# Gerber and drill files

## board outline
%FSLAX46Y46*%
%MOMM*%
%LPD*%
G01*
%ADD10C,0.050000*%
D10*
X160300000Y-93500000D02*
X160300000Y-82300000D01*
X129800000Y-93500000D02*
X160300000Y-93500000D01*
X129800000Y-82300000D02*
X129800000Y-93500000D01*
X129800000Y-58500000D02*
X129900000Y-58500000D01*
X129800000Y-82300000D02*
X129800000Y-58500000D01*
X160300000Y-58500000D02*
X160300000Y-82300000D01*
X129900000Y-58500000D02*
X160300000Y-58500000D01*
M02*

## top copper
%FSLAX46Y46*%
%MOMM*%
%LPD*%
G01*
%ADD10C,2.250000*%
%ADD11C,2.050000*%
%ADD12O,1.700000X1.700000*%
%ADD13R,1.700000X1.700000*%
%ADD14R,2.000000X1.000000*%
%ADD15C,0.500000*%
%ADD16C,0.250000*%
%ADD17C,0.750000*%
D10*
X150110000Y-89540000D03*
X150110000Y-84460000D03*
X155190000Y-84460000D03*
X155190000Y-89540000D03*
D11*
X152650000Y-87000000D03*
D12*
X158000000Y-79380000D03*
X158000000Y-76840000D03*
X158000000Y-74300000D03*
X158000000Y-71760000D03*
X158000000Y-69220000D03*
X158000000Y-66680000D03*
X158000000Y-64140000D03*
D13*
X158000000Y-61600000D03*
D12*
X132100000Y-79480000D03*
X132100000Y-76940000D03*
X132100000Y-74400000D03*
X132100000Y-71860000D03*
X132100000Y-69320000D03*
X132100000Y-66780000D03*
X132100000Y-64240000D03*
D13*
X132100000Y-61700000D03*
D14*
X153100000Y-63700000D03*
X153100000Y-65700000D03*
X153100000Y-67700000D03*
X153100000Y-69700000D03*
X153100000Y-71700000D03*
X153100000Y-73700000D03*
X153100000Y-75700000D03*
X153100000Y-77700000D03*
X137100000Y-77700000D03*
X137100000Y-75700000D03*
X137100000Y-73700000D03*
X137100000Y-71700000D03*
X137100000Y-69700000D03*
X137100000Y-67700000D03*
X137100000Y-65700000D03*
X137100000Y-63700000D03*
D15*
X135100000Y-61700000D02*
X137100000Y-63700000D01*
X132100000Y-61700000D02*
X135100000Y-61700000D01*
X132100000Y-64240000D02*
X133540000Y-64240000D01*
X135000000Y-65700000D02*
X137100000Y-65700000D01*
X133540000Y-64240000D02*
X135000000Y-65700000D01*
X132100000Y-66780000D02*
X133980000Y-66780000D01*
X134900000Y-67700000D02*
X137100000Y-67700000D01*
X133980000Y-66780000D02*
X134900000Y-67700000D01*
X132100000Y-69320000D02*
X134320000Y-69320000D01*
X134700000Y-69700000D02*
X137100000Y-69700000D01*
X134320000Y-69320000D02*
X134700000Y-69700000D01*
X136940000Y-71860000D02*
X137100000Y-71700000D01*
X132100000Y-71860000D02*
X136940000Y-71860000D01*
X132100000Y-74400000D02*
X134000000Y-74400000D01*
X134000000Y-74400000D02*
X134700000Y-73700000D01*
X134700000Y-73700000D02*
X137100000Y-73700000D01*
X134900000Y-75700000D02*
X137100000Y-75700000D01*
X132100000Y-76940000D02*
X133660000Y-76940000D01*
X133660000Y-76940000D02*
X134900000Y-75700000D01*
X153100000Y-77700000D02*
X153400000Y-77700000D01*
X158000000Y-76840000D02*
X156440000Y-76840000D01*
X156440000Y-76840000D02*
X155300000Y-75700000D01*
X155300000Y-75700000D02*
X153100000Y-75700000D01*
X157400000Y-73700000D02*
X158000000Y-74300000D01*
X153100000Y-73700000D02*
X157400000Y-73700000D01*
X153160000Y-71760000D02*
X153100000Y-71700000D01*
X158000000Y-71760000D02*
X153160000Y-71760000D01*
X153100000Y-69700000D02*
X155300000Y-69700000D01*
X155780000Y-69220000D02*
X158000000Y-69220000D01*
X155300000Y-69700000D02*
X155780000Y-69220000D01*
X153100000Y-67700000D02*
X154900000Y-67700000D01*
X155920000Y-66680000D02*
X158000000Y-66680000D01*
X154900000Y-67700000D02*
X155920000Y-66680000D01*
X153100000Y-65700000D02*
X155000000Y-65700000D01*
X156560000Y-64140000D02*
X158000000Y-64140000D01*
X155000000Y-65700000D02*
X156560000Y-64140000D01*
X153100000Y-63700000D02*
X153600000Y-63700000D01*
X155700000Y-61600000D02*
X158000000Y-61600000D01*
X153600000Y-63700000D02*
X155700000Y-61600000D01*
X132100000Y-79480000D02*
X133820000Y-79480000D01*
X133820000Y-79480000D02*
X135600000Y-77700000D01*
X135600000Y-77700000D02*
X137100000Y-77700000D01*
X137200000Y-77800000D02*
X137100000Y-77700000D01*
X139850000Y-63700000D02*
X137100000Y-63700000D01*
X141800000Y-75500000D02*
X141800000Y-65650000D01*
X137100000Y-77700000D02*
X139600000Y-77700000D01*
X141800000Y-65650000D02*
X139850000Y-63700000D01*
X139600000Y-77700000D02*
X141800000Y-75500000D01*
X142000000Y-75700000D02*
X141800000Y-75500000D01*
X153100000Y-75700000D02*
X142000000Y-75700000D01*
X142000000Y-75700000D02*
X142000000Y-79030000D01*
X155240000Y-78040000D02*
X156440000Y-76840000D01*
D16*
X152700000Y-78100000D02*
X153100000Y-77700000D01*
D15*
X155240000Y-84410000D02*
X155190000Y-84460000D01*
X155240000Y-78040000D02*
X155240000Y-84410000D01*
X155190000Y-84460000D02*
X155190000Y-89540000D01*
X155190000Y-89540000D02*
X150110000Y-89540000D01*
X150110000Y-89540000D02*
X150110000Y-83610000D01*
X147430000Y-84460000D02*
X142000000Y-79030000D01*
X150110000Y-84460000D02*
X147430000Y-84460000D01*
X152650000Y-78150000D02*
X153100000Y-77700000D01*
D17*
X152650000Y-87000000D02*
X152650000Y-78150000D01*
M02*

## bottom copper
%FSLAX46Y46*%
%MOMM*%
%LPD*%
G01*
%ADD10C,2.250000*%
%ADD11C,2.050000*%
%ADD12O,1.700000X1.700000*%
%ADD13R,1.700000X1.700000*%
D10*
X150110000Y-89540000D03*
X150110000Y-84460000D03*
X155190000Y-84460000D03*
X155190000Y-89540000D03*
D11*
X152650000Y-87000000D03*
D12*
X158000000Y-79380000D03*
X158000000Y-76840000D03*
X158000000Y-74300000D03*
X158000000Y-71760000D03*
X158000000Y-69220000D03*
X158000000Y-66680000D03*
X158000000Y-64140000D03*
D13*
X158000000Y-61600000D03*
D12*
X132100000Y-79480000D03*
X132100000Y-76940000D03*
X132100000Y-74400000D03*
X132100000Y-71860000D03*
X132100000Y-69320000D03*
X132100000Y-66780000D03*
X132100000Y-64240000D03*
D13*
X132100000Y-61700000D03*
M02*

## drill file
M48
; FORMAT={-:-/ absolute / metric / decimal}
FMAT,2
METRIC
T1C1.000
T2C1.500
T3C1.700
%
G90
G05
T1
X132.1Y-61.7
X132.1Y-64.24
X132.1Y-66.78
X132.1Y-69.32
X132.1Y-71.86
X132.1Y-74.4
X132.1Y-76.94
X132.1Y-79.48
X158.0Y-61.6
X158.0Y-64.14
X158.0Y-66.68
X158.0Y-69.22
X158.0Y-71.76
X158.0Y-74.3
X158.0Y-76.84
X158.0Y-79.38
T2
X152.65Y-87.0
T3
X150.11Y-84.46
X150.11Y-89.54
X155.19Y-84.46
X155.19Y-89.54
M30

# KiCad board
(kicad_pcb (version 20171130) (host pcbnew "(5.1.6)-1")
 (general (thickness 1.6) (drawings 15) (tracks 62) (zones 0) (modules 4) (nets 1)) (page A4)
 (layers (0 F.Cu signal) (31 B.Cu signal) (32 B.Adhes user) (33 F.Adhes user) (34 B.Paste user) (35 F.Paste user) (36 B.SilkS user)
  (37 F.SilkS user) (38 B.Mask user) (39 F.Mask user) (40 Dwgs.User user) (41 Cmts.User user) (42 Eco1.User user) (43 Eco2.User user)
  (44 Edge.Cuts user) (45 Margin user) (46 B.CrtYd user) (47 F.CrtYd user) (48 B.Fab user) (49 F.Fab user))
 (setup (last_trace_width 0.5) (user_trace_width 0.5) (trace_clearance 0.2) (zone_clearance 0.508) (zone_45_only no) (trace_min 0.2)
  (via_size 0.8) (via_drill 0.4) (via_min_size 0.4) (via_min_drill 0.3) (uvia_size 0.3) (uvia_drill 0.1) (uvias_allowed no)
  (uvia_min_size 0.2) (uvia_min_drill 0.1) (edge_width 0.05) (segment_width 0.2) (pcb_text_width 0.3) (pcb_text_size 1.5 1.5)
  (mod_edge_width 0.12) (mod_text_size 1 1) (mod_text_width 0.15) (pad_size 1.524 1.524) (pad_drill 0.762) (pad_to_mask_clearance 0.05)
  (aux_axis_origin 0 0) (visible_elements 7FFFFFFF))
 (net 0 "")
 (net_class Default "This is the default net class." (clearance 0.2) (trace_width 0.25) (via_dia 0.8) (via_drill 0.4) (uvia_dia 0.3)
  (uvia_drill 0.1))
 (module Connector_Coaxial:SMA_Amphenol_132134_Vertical (layer F.Cu) (at 152.65 87)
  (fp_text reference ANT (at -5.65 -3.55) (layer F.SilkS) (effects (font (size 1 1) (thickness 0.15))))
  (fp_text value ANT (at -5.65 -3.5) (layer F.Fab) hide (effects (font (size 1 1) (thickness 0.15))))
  (pad 2 thru_hole circle (at -2.54 2.54) (size 2.25 2.25) (drill 1.7) (layers *.Cu *.Mask))
  (pad 2 thru_hole circle (at -2.54 -2.54) (size 2.25 2.25) (drill 1.7) (layers *.Cu *.Mask))
  (pad 2 thru_hole circle (at 2.54 -2.54) (size 2.25 2.25) (drill 1.7) (layers *.Cu *.Mask))
  (pad 2 thru_hole circle (at 2.54 2.54) (size 2.25 2.25) (drill 1.7) (layers *.Cu *.Mask))
  (pad 1 thru_hole circle (at 0 0) (size 2.05 2.05) (drill 1.5) (layers *.Cu *.Mask)))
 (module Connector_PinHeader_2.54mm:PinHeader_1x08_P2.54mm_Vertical (layer F.Cu) (at 158 61.6)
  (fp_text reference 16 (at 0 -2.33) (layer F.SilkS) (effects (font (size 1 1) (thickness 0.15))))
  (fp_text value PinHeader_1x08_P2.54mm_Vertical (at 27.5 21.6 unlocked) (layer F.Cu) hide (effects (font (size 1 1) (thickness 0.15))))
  (pad 8 thru_hole oval (at 0 17.78) (size 1.7 1.7) (drill 1) (layers *.Cu *.Mask))
  (pad 7 thru_hole oval (at 0 15.24) (size 1.7 1.7) (drill 1) (layers *.Cu *.Mask))
  (pad 6 thru_hole oval (at 0 12.7) (size 1.7 1.7) (drill 1) (layers *.Cu *.Mask))
  (pad 5 thru_hole oval (at 0 10.16) (size 1.7 1.7) (drill 1) (layers *.Cu *.Mask))
  (pad 4 thru_hole oval (at 0 7.62) (size 1.7 1.7) (drill 1) (layers *.Cu *.Mask))
  (pad 3 thru_hole oval (at 0 5.08) (size 1.7 1.7) (drill 1) (layers *.Cu *.Mask))
  (pad 2 thru_hole oval (at 0 2.54) (size 1.7 1.7) (drill 1) (layers *.Cu *.Mask))
  (pad 1 thru_hole rect (at 0 0) (size 1.7 1.7) (drill 1) (layers *.Cu *.Mask)))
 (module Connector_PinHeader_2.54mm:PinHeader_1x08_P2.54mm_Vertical (layer F.Cu) (at 132.1 61.7)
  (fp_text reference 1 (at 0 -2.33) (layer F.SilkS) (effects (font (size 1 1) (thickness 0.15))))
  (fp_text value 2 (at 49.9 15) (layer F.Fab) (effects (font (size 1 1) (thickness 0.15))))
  (pad 8 thru_hole oval (at 0 17.78) (size 1.7 1.7) (drill 1) (layers *.Cu *.Mask))
  (pad 7 thru_hole oval (at 0 15.24) (size 1.7 1.7) (drill 1) (layers *.Cu *.Mask))
  (pad 6 thru_hole oval (at 0 12.7) (size 1.7 1.7) (drill 1) (layers *.Cu *.Mask))
  (pad 5 thru_hole oval (at 0 10.16) (size 1.7 1.7) (drill 1) (layers *.Cu *.Mask))
  (pad 4 thru_hole oval (at 0 7.62) (size 1.7 1.7) (drill 1) (layers *.Cu *.Mask))
  (pad 3 thru_hole oval (at 0 5.08) (size 1.7 1.7) (drill 1) (layers *.Cu *.Mask))
  (pad 2 thru_hole oval (at 0 2.54) (size 1.7 1.7) (drill 1) (layers *.Cu *.Mask))
  (pad 1 thru_hole rect (at 0 0) (size 1.7 1.7) (drill 1) (layers *.Cu *.Mask)))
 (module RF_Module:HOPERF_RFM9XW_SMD (layer F.Cu) (at 145.1 70.7)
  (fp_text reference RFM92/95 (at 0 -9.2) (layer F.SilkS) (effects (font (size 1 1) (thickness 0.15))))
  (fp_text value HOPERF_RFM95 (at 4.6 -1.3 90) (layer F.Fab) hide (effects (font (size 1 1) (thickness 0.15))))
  (pad 16 smd rect (at 8 -7) (size 2 1) (layers F.Cu F.Paste F.Mask))
  (pad 15 smd rect (at 8 -5) (size 2 1) (layers F.Cu F.Paste F.Mask))
  (pad 14 smd rect (at 8 -3) (size 2 1) (layers F.Cu F.Paste F.Mask))
  (pad 13 smd rect (at 8 -1) (size 2 1) (layers F.Cu F.Paste F.Mask))
  (pad 12 smd rect (at 8 1) (size 2 1) (layers F.Cu F.Paste F.Mask))
  (pad 11 smd rect (at 8 3) (size 2 1) (layers F.Cu F.Paste F.Mask))
  (pad 10 smd rect (at 8 5) (size 2 1) (layers F.Cu F.Paste F.Mask))
  (pad 9 smd rect (at 8 7) (size 2 1) (layers F.Cu F.Paste F.Mask))
  (pad 8 smd rect (at -8 7) (size 2 1) (layers F.Cu F.Paste F.Mask))
  (pad 7 smd rect (at -8 5) (size 2 1) (layers F.Cu F.Paste F.Mask))
  (pad 6 smd rect (at -8 3) (size 2 1) (layers F.Cu F.Paste F.Mask))
  (pad 5 smd rect (at -8 1) (size 2 1) (layers F.Cu F.Paste F.Mask))
  (pad 4 smd rect (at -8 -1) (size 2 1) (layers F.Cu F.Paste F.Mask))
  (pad 3 smd rect (at -8 -3) (size 2 1) (layers F.Cu F.Paste F.Mask))
  (pad 2 smd rect (at -8 -5) (size 2 1) (layers F.Cu F.Paste F.Mask))
  (pad 1 smd rect (at -8 -7) (size 2 1) (layers F.Cu F.Paste F.Mask)))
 (gr_line (start 160.3 93.5) (end 160.3 82.3) (layer Edge.Cuts) (width 0.05))
 (gr_line (start 129.8 93.5) (end 160.3 93.5) (layer Edge.Cuts) (width 0.05))
 (gr_line (start 129.8 82.3) (end 129.8 93.5) (layer Edge.Cuts) (width 0.05))
 (gr_line (start 129.8 58.5) (end 129.9 58.5) (layer Edge.Cuts) (width 0.05))
 (gr_line (start 129.8 82.3) (end 129.8 58.5) (layer Edge.Cuts) (width 0.05))
 (gr_line (start 160.3 58.5) (end 160.3 82.3) (layer Edge.Cuts) (width 0.05))
 (gr_line (start 129.9 58.5) (end 160.3 58.5) (layer Edge.Cuts) (width 0.05))
 (segment (start 135.1 61.7) (end 137.1 63.7) (width 0.5) (layer F.Cu) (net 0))
 (segment (start 132.1 61.7) (end 135.1 61.7) (width 0.5) (layer F.Cu) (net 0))
 (segment (start 132.1 64.24) (end 133.54 64.24) (width 0.5) (layer F.Cu) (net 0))
 (segment (start 135 65.7) (end 137.1 65.7) (width 0.5) (layer F.Cu) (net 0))
 (segment (start 133.54 64.24) (end 135 65.7) (width 0.5) (layer F.Cu) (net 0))
 (segment (start 132.1 66.78) (end 133.98 66.78) (width 0.5) (layer F.Cu) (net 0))
 (segment (start 134.9 67.7) (end 137.1 67.7) (width 0.5) (layer F.Cu) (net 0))
 (segment (start 133.98 66.78) (end 134.9 67.7) (width 0.5) (layer F.Cu) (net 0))
 (segment (start 132.1 69.32) (end 134.32 69.32) (width 0.5) (layer F.Cu) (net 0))
 (segment (start 134.7 69.7) (end 137.1 69.7) (width 0.5) (layer F.Cu) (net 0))
 (segment (start 134.32 69.32) (end 134.7 69.7) (width 0.5) (layer F.Cu) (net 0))
 (segment (start 136.94 71.86) (end 137.1 71.7) (width 0.5) (layer F.Cu) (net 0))
 (segment (start 132.1 71.86) (end 136.94 71.86) (width 0.5) (layer F.Cu) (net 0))
 (segment (start 132.1 74.4) (end 134 74.4) (width 0.5) (layer F.Cu) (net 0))
 (segment (start 134 74.4) (end 134.7 73.7) (width 0.5) (layer F.Cu) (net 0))
 (segment (start 134.7 73.7) (end 137.1 73.7) (width 0.5) (layer F.Cu) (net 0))
 (segment (start 134.9 75.7) (end 137.1 75.7) (width 0.5) (layer F.Cu) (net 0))
 (segment (start 132.1 76.94) (end 133.66 76.94) (width 0.5) (layer F.Cu) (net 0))
 (segment (start 133.66 76.94) (end 134.9 75.7) (width 0.5) (layer F.Cu) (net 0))
 (segment (start 153.1 77.7) (end 153.4 77.7) (width 0.5) (layer F.Cu) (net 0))
 (segment (start 158 76.84) (end 156.44 76.84) (width 0.5) (layer F.Cu) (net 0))
 (segment (start 156.44 76.84) (end 155.3 75.7) (width 0.5) (layer F.Cu) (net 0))
 (segment (start 155.3 75.7) (end 153.1 75.7) (width 0.5) (layer F.Cu) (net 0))
 (segment (start 157.4 73.7) (end 158 74.3) (width 0.5) (layer F.Cu) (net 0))
 (segment (start 153.1 73.7) (end 157.4 73.7) (width 0.5) (layer F.Cu) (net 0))
 (segment (start 153.16 71.76) (end 153.1 71.7) (width 0.5) (layer F.Cu) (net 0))
 (segment (start 158 71.76) (end 153.16 71.76) (width 0.5) (layer F.Cu) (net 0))
 (segment (start 153.1 69.7) (end 155.3 69.7) (width 0.5) (layer F.Cu) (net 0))
 (segment (start 155.78 69.22) (end 158 69.22) (width 0.5) (layer F.Cu) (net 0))
 (segment (start 155.3 69.7) (end 155.78 69.22) (width 0.5) (layer F.Cu) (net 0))
 (segment (start 153.1 67.7) (end 154.9 67.7) (width 0.5) (layer F.Cu) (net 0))
 (segment (start 155.92 66.68) (end 158 66.68) (width 0.5) (layer F.Cu) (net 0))
 (segment (start 154.9 67.7) (end 155.92 66.68) (width 0.5) (layer F.Cu) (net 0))
 (segment (start 153.1 65.7) (end 155 65.7) (width 0.5) (layer F.Cu) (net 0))
 (segment (start 156.56 64.14) (end 158 64.14) (width 0.5) (layer F.Cu) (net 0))
 (segment (start 155 65.7) (end 156.56 64.14) (width 0.5) (layer F.Cu) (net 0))
 (segment (start 153.1 63.7) (end 153.6 63.7) (width 0.5) (layer F.Cu) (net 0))
 (segment (start 155.7 61.6) (end 158 61.6) (width 0.5) (layer F.Cu) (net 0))
 (segment (start 153.6 63.7) (end 155.7 61.6) (width 0.5) (layer F.Cu) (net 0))
 (segment (start 132.1 79.48) (end 133.82 79.48) (width 0.5) (layer F.Cu) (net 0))
 (segment (start 133.82 79.48) (end 135.6 77.7) (width 0.5) (layer F.Cu) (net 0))
 (segment (start 135.6 77.7) (end 137.1 77.7) (width 0.5) (layer F.Cu) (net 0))
 (segment (start 137.2 77.8) (end 137.1 77.7) (width 0.5) (layer F.Cu) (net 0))
 (segment (start 139.85 63.7) (end 137.1 63.7) (width 0.5) (layer F.Cu) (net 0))
 (segment (start 141.8 75.5) (end 141.8 65.65) (width 0.5) (layer F.Cu) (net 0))
 (segment (start 137.1 77.7) (end 139.6 77.7) (width 0.5) (layer F.Cu) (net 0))
 (segment (start 141.8 65.65) (end 139.85 63.7) (width 0.5) (layer F.Cu) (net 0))
 (segment (start 139.6 77.7) (end 141.8 75.5) (width 0.5) (layer F.Cu) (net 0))
 (segment (start 142 75.7) (end 141.8 75.5) (width 0.5) (layer F.Cu) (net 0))
 (segment (start 153.1 75.7) (end 142 75.7) (width 0.5) (layer F.Cu) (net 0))
 (segment (start 142 75.7) (end 142 79.03) (width 0.5) (layer F.Cu) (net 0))
 (segment (start 155.24 78.04) (end 156.44 76.84) (width 0.5) (layer F.Cu) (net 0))
 (segment (start 152.7 78.1) (end 153.1 77.7) (width 0.25) (layer F.Cu) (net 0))
 (segment (start 155.24 84.41) (end 155.19 84.46) (width 0.5) (layer F.Cu) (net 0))
 (segment (start 155.24 78.04) (end 155.24 84.41) (width 0.5) (layer F.Cu) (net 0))
 (segment (start 155.19 84.46) (end 155.19 89.54) (width 0.5) (layer F.Cu) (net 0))
 (segment (start 155.19 89.54) (end 150.11 89.54) (width 0.5) (layer F.Cu) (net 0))
 (segment (start 150.11 89.54) (end 150.11 83.61) (width 0.5) (layer F.Cu) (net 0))
 (segment (start 147.43 84.46) (end 142 79.03) (width 0.5) (layer F.Cu) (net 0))
 (segment (start 150.11 84.46) (end 147.43 84.46) (width 0.5) (layer F.Cu) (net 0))
 (segment (start 152.65 78.15) (end 153.1 77.7) (width 0.5) (layer F.Cu) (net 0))
 (segment (start 152.65 87) (end 152.65 78.15) (width 0.75) (layer F.Cu) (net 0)))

